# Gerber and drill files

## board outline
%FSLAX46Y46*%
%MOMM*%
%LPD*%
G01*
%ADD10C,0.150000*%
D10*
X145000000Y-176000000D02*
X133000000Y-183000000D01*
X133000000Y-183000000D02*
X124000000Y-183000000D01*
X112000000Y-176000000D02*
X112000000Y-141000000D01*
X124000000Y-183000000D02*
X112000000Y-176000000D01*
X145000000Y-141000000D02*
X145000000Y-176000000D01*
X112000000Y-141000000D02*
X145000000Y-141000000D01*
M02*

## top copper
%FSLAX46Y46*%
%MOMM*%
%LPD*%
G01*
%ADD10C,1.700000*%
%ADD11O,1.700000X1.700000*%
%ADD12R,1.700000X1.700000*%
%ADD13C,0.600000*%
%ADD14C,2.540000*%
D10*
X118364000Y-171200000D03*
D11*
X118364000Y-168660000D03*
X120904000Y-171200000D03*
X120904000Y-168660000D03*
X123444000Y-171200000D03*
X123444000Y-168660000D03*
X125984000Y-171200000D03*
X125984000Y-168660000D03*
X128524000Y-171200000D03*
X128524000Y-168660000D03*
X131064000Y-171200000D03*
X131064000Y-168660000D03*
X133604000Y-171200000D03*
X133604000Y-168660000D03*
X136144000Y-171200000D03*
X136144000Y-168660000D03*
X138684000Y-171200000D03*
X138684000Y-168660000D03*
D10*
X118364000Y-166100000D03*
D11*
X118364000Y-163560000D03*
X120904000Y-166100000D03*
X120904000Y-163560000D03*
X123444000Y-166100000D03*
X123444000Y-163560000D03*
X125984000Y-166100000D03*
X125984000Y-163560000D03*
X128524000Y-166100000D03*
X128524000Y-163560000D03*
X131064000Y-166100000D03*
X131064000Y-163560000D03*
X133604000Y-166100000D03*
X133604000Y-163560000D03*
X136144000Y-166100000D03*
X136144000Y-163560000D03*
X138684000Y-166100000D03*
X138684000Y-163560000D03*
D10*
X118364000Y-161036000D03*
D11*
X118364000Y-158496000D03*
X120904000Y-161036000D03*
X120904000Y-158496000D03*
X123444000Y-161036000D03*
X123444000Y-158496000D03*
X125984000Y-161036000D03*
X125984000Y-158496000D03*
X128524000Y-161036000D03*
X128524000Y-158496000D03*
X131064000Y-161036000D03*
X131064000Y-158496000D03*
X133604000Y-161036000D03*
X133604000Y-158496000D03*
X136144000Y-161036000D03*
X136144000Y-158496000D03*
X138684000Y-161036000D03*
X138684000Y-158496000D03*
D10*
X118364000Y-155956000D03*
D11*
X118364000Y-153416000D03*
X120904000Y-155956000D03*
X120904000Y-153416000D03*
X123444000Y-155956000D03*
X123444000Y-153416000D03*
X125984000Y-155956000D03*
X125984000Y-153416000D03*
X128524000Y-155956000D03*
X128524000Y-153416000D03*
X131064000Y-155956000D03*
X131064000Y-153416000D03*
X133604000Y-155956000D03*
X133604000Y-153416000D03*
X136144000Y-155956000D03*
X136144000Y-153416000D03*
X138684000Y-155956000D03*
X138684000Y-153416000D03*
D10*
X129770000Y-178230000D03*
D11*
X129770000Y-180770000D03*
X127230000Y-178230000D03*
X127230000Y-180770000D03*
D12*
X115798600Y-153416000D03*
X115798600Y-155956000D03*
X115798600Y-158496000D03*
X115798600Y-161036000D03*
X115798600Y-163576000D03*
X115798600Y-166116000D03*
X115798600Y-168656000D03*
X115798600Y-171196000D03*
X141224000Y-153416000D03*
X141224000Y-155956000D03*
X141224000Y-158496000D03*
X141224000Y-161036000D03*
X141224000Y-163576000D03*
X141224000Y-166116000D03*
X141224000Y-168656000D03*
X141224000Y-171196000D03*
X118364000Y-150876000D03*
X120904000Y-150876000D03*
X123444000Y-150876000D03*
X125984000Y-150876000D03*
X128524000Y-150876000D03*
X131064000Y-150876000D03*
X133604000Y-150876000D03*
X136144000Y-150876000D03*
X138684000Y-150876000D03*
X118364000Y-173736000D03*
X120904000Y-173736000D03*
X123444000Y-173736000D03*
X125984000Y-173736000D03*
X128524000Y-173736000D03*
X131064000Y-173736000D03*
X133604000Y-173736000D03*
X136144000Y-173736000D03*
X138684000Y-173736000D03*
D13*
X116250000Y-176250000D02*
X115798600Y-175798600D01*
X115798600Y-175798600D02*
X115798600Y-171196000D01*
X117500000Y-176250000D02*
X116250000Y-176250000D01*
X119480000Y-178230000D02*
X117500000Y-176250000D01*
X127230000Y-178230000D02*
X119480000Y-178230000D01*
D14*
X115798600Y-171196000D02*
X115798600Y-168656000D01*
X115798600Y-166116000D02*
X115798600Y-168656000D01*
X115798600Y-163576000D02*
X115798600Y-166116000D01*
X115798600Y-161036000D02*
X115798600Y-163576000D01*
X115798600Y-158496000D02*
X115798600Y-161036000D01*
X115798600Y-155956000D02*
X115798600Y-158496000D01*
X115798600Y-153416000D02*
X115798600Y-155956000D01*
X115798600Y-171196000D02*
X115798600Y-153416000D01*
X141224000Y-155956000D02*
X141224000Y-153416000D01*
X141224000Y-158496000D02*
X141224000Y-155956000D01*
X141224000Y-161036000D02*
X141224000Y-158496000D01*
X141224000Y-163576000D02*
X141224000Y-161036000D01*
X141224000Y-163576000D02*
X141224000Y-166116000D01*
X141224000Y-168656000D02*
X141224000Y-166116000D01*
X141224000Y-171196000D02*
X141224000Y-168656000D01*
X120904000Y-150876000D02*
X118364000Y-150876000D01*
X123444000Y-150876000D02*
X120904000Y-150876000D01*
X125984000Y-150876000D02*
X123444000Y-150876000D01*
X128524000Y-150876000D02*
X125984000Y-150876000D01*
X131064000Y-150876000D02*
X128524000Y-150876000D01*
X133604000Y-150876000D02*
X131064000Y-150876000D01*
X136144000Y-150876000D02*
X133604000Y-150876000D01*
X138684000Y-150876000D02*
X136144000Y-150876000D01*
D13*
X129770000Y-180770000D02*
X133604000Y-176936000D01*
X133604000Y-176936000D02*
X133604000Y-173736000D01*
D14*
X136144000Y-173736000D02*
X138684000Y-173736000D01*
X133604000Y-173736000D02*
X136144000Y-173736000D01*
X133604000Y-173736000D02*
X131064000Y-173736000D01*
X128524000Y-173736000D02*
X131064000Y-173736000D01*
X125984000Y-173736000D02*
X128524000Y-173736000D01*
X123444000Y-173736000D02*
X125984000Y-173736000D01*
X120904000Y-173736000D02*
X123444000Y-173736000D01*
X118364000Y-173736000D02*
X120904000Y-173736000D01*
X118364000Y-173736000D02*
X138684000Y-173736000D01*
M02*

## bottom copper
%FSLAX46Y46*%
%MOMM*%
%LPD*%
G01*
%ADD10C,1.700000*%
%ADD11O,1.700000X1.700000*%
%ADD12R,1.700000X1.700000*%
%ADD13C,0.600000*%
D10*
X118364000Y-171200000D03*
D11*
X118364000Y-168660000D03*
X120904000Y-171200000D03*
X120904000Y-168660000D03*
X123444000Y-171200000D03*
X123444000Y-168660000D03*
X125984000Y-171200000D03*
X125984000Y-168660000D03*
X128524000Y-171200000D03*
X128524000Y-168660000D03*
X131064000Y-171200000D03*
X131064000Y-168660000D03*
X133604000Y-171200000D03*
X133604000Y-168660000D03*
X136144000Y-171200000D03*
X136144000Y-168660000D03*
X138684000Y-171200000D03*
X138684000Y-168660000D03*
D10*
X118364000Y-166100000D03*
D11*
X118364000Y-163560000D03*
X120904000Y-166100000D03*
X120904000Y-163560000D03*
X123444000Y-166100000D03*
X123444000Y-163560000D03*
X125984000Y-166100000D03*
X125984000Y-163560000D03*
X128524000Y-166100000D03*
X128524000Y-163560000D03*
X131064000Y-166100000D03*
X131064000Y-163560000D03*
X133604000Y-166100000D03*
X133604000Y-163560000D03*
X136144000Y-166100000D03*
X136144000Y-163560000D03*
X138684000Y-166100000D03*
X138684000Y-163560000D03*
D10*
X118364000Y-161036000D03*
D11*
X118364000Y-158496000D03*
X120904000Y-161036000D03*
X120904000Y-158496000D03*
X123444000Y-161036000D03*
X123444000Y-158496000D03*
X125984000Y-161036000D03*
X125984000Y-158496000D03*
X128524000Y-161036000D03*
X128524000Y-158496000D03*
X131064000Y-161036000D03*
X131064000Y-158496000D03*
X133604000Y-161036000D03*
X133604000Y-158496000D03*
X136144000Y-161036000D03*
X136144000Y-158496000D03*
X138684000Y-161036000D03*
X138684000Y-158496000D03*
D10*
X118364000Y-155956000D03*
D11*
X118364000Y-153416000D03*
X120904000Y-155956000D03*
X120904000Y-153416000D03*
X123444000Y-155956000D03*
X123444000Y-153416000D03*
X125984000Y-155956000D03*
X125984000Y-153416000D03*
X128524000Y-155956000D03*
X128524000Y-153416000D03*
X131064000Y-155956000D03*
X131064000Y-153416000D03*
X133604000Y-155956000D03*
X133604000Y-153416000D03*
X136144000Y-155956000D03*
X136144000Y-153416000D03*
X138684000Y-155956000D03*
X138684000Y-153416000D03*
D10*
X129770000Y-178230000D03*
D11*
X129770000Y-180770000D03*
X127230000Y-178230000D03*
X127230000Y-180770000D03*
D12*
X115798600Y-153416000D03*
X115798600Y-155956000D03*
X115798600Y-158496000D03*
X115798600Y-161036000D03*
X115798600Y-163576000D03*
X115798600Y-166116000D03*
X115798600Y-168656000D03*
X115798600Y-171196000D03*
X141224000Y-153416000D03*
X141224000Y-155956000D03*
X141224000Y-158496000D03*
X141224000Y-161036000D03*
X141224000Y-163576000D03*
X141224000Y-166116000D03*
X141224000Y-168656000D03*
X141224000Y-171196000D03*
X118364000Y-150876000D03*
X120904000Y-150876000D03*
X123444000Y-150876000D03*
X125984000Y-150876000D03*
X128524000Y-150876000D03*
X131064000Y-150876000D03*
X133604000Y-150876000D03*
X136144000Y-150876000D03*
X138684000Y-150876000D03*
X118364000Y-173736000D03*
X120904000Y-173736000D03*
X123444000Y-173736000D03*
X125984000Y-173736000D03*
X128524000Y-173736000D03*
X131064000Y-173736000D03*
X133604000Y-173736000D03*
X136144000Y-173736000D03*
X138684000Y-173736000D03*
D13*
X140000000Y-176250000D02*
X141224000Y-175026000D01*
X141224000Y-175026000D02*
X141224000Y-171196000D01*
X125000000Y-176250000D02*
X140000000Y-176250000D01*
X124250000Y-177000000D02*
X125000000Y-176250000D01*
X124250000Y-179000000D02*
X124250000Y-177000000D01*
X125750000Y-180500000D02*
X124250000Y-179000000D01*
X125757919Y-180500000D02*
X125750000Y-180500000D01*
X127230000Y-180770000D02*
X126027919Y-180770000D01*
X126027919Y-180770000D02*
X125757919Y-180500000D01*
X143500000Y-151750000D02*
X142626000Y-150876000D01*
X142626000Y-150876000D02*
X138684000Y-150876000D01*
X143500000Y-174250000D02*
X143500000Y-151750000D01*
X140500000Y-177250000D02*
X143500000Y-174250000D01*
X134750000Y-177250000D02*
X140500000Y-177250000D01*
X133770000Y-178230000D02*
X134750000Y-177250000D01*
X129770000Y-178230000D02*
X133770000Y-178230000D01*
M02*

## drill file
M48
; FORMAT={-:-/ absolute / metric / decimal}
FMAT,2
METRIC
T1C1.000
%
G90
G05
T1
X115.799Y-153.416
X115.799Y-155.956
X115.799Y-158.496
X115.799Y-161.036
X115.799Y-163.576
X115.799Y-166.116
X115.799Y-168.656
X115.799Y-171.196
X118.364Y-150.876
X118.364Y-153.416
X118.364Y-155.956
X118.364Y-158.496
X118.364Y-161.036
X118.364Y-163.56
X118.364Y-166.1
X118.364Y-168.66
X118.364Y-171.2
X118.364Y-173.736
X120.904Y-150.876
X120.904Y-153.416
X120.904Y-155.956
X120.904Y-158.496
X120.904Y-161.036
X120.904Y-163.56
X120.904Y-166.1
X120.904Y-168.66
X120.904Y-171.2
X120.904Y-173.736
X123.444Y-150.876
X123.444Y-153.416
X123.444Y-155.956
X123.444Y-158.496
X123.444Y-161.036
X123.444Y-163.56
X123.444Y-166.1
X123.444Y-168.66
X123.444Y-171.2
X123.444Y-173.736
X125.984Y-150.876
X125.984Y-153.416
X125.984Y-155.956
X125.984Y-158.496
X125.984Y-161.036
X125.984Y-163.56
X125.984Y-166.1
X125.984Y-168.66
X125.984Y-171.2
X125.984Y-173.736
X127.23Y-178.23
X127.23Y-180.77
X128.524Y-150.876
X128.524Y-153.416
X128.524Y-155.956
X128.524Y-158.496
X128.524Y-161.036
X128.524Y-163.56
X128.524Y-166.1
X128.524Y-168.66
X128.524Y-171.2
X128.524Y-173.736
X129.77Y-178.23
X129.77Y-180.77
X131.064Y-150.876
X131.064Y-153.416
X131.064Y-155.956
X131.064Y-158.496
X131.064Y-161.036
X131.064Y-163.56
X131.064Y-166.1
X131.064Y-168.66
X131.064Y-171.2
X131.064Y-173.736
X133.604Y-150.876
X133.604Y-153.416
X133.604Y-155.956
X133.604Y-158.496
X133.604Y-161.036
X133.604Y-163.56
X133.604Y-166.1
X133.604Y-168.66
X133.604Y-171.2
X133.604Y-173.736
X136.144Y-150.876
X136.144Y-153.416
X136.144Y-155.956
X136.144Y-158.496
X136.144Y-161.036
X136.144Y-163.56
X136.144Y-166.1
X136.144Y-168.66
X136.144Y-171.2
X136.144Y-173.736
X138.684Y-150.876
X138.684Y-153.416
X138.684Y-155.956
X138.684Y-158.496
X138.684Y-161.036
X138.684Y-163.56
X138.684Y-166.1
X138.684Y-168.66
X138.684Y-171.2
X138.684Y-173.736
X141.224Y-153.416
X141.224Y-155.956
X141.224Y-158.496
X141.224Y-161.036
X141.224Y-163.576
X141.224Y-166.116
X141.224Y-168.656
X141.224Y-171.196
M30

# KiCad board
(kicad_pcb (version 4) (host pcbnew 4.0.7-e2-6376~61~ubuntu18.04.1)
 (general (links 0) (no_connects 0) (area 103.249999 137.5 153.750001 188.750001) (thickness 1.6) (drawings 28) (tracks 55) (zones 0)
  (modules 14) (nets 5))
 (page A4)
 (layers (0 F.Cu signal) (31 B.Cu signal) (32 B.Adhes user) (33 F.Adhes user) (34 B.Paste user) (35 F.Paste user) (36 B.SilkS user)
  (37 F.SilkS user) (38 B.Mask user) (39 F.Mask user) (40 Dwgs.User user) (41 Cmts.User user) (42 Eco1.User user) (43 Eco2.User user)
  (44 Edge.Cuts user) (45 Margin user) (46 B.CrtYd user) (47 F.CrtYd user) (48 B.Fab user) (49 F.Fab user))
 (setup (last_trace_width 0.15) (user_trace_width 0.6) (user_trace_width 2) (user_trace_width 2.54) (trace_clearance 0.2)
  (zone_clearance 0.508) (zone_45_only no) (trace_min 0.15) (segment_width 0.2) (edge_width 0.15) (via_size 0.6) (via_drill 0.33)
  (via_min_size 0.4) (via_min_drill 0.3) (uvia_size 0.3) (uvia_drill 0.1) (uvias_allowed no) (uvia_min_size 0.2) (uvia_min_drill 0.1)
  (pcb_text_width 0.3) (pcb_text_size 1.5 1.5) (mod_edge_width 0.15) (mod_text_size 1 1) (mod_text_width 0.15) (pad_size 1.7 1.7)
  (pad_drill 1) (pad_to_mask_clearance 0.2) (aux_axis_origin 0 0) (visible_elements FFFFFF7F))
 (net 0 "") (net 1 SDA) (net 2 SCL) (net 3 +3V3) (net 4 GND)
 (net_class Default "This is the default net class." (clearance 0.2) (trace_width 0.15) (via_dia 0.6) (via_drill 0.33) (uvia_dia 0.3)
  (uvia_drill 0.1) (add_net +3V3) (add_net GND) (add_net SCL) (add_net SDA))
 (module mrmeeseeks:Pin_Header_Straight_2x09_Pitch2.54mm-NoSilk (layer F.Cu) (at 118.364 171.2 90)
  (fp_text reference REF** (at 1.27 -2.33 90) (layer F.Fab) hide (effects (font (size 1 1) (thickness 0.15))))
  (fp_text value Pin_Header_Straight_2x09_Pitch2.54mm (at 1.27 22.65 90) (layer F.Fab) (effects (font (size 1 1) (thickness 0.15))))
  (pad 1 thru_hole circle (at 0 0 90) (size 1.7 1.7) (drill 1) (layers *.Cu *.Mask))
  (pad 2 thru_hole oval (at 2.54 0 90) (size 1.7 1.7) (drill 1) (layers *.Cu *.Mask))
  (pad 3 thru_hole oval (at 0 2.54 90) (size 1.7 1.7) (drill 1) (layers *.Cu *.Mask))
  (pad 4 thru_hole oval (at 2.54 2.54 90) (size 1.7 1.7) (drill 1) (layers *.Cu *.Mask))
  (pad 5 thru_hole oval (at 0 5.08 90) (size 1.7 1.7) (drill 1) (layers *.Cu *.Mask))
  (pad 6 thru_hole oval (at 2.54 5.08 90) (size 1.7 1.7) (drill 1) (layers *.Cu *.Mask))
  (pad 7 thru_hole oval (at 0 7.62 90) (size 1.7 1.7) (drill 1) (layers *.Cu *.Mask))
  (pad 8 thru_hole oval (at 2.54 7.62 90) (size 1.7 1.7) (drill 1) (layers *.Cu *.Mask))
  (pad 9 thru_hole oval (at 0 10.16 90) (size 1.7 1.7) (drill 1) (layers *.Cu *.Mask))
  (pad 10 thru_hole oval (at 2.54 10.16 90) (size 1.7 1.7) (drill 1) (layers *.Cu *.Mask))
  (pad 11 thru_hole oval (at 0 12.7 90) (size 1.7 1.7) (drill 1) (layers *.Cu *.Mask))
  (pad 12 thru_hole oval (at 2.54 12.7 90) (size 1.7 1.7) (drill 1) (layers *.Cu *.Mask))
  (pad 13 thru_hole oval (at 0 15.24 90) (size 1.7 1.7) (drill 1) (layers *.Cu *.Mask))
  (pad 14 thru_hole oval (at 2.54 15.24 90) (size 1.7 1.7) (drill 1) (layers *.Cu *.Mask))
  (pad 15 thru_hole oval (at 0 17.78 90) (size 1.7 1.7) (drill 1) (layers *.Cu *.Mask))
  (pad 16 thru_hole oval (at 2.54 17.78 90) (size 1.7 1.7) (drill 1) (layers *.Cu *.Mask))
  (pad 17 thru_hole oval (at 0 20.32 90) (size 1.7 1.7) (drill 1) (layers *.Cu *.Mask))
  (pad 18 thru_hole oval (at 2.54 20.32 90) (size 1.7 1.7) (drill 1) (layers *.Cu *.Mask)))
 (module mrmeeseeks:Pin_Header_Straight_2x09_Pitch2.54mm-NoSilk (layer F.Cu) (at 118.364 166.1 90)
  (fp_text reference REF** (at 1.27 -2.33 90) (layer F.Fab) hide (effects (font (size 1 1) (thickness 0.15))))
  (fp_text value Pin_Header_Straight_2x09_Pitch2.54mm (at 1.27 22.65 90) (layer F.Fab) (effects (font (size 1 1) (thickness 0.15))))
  (pad 1 thru_hole circle (at 0 0 90) (size 1.7 1.7) (drill 1) (layers *.Cu *.Mask))
  (pad 2 thru_hole oval (at 2.54 0 90) (size 1.7 1.7) (drill 1) (layers *.Cu *.Mask))
  (pad 3 thru_hole oval (at 0 2.54 90) (size 1.7 1.7) (drill 1) (layers *.Cu *.Mask))
  (pad 4 thru_hole oval (at 2.54 2.54 90) (size 1.7 1.7) (drill 1) (layers *.Cu *.Mask))
  (pad 5 thru_hole oval (at 0 5.08 90) (size 1.7 1.7) (drill 1) (layers *.Cu *.Mask))
  (pad 6 thru_hole oval (at 2.54 5.08 90) (size 1.7 1.7) (drill 1) (layers *.Cu *.Mask))
  (pad 7 thru_hole oval (at 0 7.62 90) (size 1.7 1.7) (drill 1) (layers *.Cu *.Mask))
  (pad 8 thru_hole oval (at 2.54 7.62 90) (size 1.7 1.7) (drill 1) (layers *.Cu *.Mask))
  (pad 9 thru_hole oval (at 0 10.16 90) (size 1.7 1.7) (drill 1) (layers *.Cu *.Mask))
  (pad 10 thru_hole oval (at 2.54 10.16 90) (size 1.7 1.7) (drill 1) (layers *.Cu *.Mask))
  (pad 11 thru_hole oval (at 0 12.7 90) (size 1.7 1.7) (drill 1) (layers *.Cu *.Mask))
  (pad 12 thru_hole oval (at 2.54 12.7 90) (size 1.7 1.7) (drill 1) (layers *.Cu *.Mask))
  (pad 13 thru_hole oval (at 0 15.24 90) (size 1.7 1.7) (drill 1) (layers *.Cu *.Mask))
  (pad 14 thru_hole oval (at 2.54 15.24 90) (size 1.7 1.7) (drill 1) (layers *.Cu *.Mask))
  (pad 15 thru_hole oval (at 0 17.78 90) (size 1.7 1.7) (drill 1) (layers *.Cu *.Mask))
  (pad 16 thru_hole oval (at 2.54 17.78 90) (size 1.7 1.7) (drill 1) (layers *.Cu *.Mask))
  (pad 17 thru_hole oval (at 0 20.32 90) (size 1.7 1.7) (drill 1) (layers *.Cu *.Mask))
  (pad 18 thru_hole oval (at 2.54 20.32 90) (size 1.7 1.7) (drill 1) (layers *.Cu *.Mask)))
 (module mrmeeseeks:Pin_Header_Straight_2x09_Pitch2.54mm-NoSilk (layer F.Cu) (at 118.364 161.036 90)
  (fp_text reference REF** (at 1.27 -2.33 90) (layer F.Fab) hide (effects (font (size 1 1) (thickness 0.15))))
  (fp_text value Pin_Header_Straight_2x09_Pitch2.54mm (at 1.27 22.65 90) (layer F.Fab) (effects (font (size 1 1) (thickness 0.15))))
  (pad 1 thru_hole circle (at 0 0 90) (size 1.7 1.7) (drill 1) (layers *.Cu *.Mask))
  (pad 2 thru_hole oval (at 2.54 0 90) (size 1.7 1.7) (drill 1) (layers *.Cu *.Mask))
  (pad 3 thru_hole oval (at 0 2.54 90) (size 1.7 1.7) (drill 1) (layers *.Cu *.Mask))
  (pad 4 thru_hole oval (at 2.54 2.54 90) (size 1.7 1.7) (drill 1) (layers *.Cu *.Mask))
  (pad 5 thru_hole oval (at 0 5.08 90) (size 1.7 1.7) (drill 1) (layers *.Cu *.Mask))
  (pad 6 thru_hole oval (at 2.54 5.08 90) (size 1.7 1.7) (drill 1) (layers *.Cu *.Mask))
  (pad 7 thru_hole oval (at 0 7.62 90) (size 1.7 1.7) (drill 1) (layers *.Cu *.Mask))
  (pad 8 thru_hole oval (at 2.54 7.62 90) (size 1.7 1.7) (drill 1) (layers *.Cu *.Mask))
  (pad 9 thru_hole oval (at 0 10.16 90) (size 1.7 1.7) (drill 1) (layers *.Cu *.Mask))
  (pad 10 thru_hole oval (at 2.54 10.16 90) (size 1.7 1.7) (drill 1) (layers *.Cu *.Mask))
  (pad 11 thru_hole oval (at 0 12.7 90) (size 1.7 1.7) (drill 1) (layers *.Cu *.Mask))
  (pad 12 thru_hole oval (at 2.54 12.7 90) (size 1.7 1.7) (drill 1) (layers *.Cu *.Mask))
  (pad 13 thru_hole oval (at 0 15.24 90) (size 1.7 1.7) (drill 1) (layers *.Cu *.Mask))
  (pad 14 thru_hole oval (at 2.54 15.24 90) (size 1.7 1.7) (drill 1) (layers *.Cu *.Mask))
  (pad 15 thru_hole oval (at 0 17.78 90) (size 1.7 1.7) (drill 1) (layers *.Cu *.Mask))
  (pad 16 thru_hole oval (at 2.54 17.78 90) (size 1.7 1.7) (drill 1) (layers *.Cu *.Mask))
  (pad 17 thru_hole oval (at 0 20.32 90) (size 1.7 1.7) (drill 1) (layers *.Cu *.Mask))
  (pad 18 thru_hole oval (at 2.54 20.32 90) (size 1.7 1.7) (drill 1) (layers *.Cu *.Mask)))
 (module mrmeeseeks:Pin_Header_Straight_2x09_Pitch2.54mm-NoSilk (layer F.Cu) (at 118.364 155.956 90)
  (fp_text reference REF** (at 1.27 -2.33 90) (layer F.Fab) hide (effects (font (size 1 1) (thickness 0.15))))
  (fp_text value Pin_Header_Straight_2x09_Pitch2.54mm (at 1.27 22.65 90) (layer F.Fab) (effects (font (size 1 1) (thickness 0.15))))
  (pad 1 thru_hole circle (at 0 0 90) (size 1.7 1.7) (drill 1) (layers *.Cu *.Mask))
  (pad 2 thru_hole oval (at 2.54 0 90) (size 1.7 1.7) (drill 1) (layers *.Cu *.Mask))
  (pad 3 thru_hole oval (at 0 2.54 90) (size 1.7 1.7) (drill 1) (layers *.Cu *.Mask))
  (pad 4 thru_hole oval (at 2.54 2.54 90) (size 1.7 1.7) (drill 1) (layers *.Cu *.Mask))
  (pad 5 thru_hole oval (at 0 5.08 90) (size 1.7 1.7) (drill 1) (layers *.Cu *.Mask))
  (pad 6 thru_hole oval (at 2.54 5.08 90) (size 1.7 1.7) (drill 1) (layers *.Cu *.Mask))
  (pad 7 thru_hole oval (at 0 7.62 90) (size 1.7 1.7) (drill 1) (layers *.Cu *.Mask))
  (pad 8 thru_hole oval (at 2.54 7.62 90) (size 1.7 1.7) (drill 1) (layers *.Cu *.Mask))
  (pad 9 thru_hole oval (at 0 10.16 90) (size 1.7 1.7) (drill 1) (layers *.Cu *.Mask))
  (pad 10 thru_hole oval (at 2.54 10.16 90) (size 1.7 1.7) (drill 1) (layers *.Cu *.Mask))
  (pad 11 thru_hole oval (at 0 12.7 90) (size 1.7 1.7) (drill 1) (layers *.Cu *.Mask))
  (pad 12 thru_hole oval (at 2.54 12.7 90) (size 1.7 1.7) (drill 1) (layers *.Cu *.Mask))
  (pad 13 thru_hole oval (at 0 15.24 90) (size 1.7 1.7) (drill 1) (layers *.Cu *.Mask))
  (pad 14 thru_hole oval (at 2.54 15.24 90) (size 1.7 1.7) (drill 1) (layers *.Cu *.Mask))
  (pad 15 thru_hole oval (at 0 17.78 90) (size 1.7 1.7) (drill 1) (layers *.Cu *.Mask))
  (pad 16 thru_hole oval (at 2.54 17.78 90) (size 1.7 1.7) (drill 1) (layers *.Cu *.Mask))
  (pad 17 thru_hole oval (at 0 20.32 90) (size 1.7 1.7) (drill 1) (layers *.Cu *.Mask))
  (pad 18 thru_hole oval (at 2.54 20.32 90) (size 1.7 1.7) (drill 1) (layers *.Cu *.Mask)))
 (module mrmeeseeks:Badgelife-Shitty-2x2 (layer F.Cu) (at 128.5 179.5)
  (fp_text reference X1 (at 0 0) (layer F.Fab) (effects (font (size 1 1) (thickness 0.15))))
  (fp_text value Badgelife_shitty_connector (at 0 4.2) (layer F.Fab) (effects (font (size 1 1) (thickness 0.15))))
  (pad 4 thru_hole circle (at 1.27 -1.27) (size 1.7 1.7) (drill 1) (layers *.Cu *.Mask) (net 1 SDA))
  (pad 3 thru_hole oval (at 1.27 1.27) (size 1.7 1.7) (drill 1) (layers *.Cu *.Mask) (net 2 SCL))
  (pad 1 thru_hole oval (at -1.27 -1.27) (size 1.7 1.7) (drill 1) (layers *.Cu *.Mask) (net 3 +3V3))
  (pad 2 thru_hole oval (at -1.27 1.27) (size 1.7 1.7) (drill 1) (layers *.Cu *.Mask) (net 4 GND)))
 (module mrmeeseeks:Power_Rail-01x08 (layer F.Cu) (at 115.7986 153.416)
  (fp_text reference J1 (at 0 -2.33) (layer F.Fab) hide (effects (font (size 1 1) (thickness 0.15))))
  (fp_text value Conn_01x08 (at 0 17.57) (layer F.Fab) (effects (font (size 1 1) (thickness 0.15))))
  (pad 1 thru_hole rect (at 0 0) (size 1.7 1.7) (drill 1) (layers *.Cu *.Mask) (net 3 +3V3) (solder_mask_margin 0.1))
  (pad 2 thru_hole rect (at 0 2.54) (size 1.7 1.7) (drill 1) (layers *.Cu *.Mask) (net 3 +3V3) (solder_mask_margin 0.1))
  (pad 3 thru_hole rect (at 0 5.08) (size 1.7 1.7) (drill 1) (layers *.Cu *.Mask) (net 3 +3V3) (solder_mask_margin 0.1))
  (pad 4 thru_hole rect (at 0 7.62) (size 1.7 1.7) (drill 1) (layers *.Cu *.Mask) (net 3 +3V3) (solder_mask_margin 0.1))
  (pad 5 thru_hole rect (at 0 10.16) (size 1.7 1.7) (drill 1) (layers *.Cu *.Mask) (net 3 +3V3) (solder_mask_margin 0.1))
  (pad 6 thru_hole rect (at 0 12.7) (size 1.7 1.7) (drill 1) (layers *.Cu *.Mask) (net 3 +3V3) (solder_mask_margin 0.1))
  (pad 7 thru_hole rect (at 0 15.24) (size 1.7 1.7) (drill 1) (layers *.Cu *.Mask) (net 3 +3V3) (solder_mask_margin 0.1))
  (pad 8 thru_hole rect (at 0 17.78) (size 1.7 1.7) (drill 1) (layers *.Cu *.Mask) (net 3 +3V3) (solder_mask_margin 0.1)))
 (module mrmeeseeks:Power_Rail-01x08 (layer F.Cu) (at 141.224 153.416)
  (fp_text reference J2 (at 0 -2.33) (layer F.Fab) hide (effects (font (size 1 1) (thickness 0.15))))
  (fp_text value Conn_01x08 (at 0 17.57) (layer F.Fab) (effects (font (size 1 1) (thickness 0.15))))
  (pad 1 thru_hole rect (at 0 0) (size 1.7 1.7) (drill 1) (layers *.Cu *.Mask) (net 4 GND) (solder_mask_margin 0.1))
  (pad 2 thru_hole rect (at 0 2.54) (size 1.7 1.7) (drill 1) (layers *.Cu *.Mask) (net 4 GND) (solder_mask_margin 0.1))
  (pad 3 thru_hole rect (at 0 5.08) (size 1.7 1.7) (drill 1) (layers *.Cu *.Mask) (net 4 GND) (solder_mask_margin 0.1))
  (pad 4 thru_hole rect (at 0 7.62) (size 1.7 1.7) (drill 1) (layers *.Cu *.Mask) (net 4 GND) (solder_mask_margin 0.1))
  (pad 5 thru_hole rect (at 0 10.16) (size 1.7 1.7) (drill 1) (layers *.Cu *.Mask) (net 4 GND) (solder_mask_margin 0.1))
  (pad 6 thru_hole rect (at 0 12.7) (size 1.7 1.7) (drill 1) (layers *.Cu *.Mask) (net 4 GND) (solder_mask_margin 0.1))
  (pad 7 thru_hole rect (at 0 15.24) (size 1.7 1.7) (drill 1) (layers *.Cu *.Mask) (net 4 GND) (solder_mask_margin 0.1))
  (pad 8 thru_hole rect (at 0 17.78) (size 1.7 1.7) (drill 1) (layers *.Cu *.Mask) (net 4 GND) (solder_mask_margin 0.1)))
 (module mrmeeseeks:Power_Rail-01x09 (layer F.Cu) (at 118.364 150.876 90)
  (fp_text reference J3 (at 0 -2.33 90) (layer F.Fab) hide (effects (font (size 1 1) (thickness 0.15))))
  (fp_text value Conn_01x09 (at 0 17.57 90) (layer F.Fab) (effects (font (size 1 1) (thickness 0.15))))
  (pad 1 thru_hole rect (at 0 0 90) (size 1.7 1.7) (drill 1) (layers *.Cu *.Mask) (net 1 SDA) (solder_mask_margin 0.1))
  (pad 2 thru_hole rect (at 0 2.54 90) (size 1.7 1.7) (drill 1) (layers *.Cu *.Mask) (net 1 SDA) (solder_mask_margin 0.1))
  (pad 3 thru_hole rect (at 0 5.08 90) (size 1.7 1.7) (drill 1) (layers *.Cu *.Mask) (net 1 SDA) (solder_mask_margin 0.1))
  (pad 4 thru_hole rect (at 0 7.62 90) (size 1.7 1.7) (drill 1) (layers *.Cu *.Mask) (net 1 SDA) (solder_mask_margin 0.1))
  (pad 5 thru_hole rect (at 0 10.16 90) (size 1.7 1.7) (drill 1) (layers *.Cu *.Mask) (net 1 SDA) (solder_mask_margin 0.1))
  (pad 6 thru_hole rect (at 0 12.7 90) (size 1.7 1.7) (drill 1) (layers *.Cu *.Mask) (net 1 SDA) (solder_mask_margin 0.1))
  (pad 7 thru_hole rect (at 0 15.24 90) (size 1.7 1.7) (drill 1) (layers *.Cu *.Mask) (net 1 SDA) (solder_mask_margin 0.1))
  (pad 8 thru_hole rect (at 0 17.78 90) (size 1.7 1.7) (drill 1) (layers *.Cu *.Mask) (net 1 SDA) (solder_mask_margin 0.1))
  (pad 9 thru_hole rect (at 0 20.32 90) (size 1.7 1.7) (drill 1) (layers *.Cu *.Mask) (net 1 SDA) (solder_mask_margin 0.1)))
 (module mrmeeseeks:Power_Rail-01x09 (layer F.Cu) (at 118.364 173.736 90)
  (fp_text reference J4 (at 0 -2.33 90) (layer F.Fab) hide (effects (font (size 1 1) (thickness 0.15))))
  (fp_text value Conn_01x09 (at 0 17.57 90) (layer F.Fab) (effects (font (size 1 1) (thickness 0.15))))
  (pad 1 thru_hole rect (at 0 0 90) (size 1.7 1.7) (drill 1) (layers *.Cu *.Mask) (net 2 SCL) (solder_mask_margin 0.1))
  (pad 2 thru_hole rect (at 0 2.54 90) (size 1.7 1.7) (drill 1) (layers *.Cu *.Mask) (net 2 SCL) (solder_mask_margin 0.1))
  (pad 3 thru_hole rect (at 0 5.08 90) (size 1.7 1.7) (drill 1) (layers *.Cu *.Mask) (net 2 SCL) (solder_mask_margin 0.1))
  (pad 4 thru_hole rect (at 0 7.62 90) (size 1.7 1.7) (drill 1) (layers *.Cu *.Mask) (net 2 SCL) (solder_mask_margin 0.1))
  (pad 5 thru_hole rect (at 0 10.16 90) (size 1.7 1.7) (drill 1) (layers *.Cu *.Mask) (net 2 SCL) (solder_mask_margin 0.1))
  (pad 6 thru_hole rect (at 0 12.7 90) (size 1.7 1.7) (drill 1) (layers *.Cu *.Mask) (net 2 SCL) (solder_mask_margin 0.1))
  (pad 7 thru_hole rect (at 0 15.24 90) (size 1.7 1.7) (drill 1) (layers *.Cu *.Mask) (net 2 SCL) (solder_mask_margin 0.1))
  (pad 8 thru_hole rect (at 0 17.78 90) (size 1.7 1.7) (drill 1) (layers *.Cu *.Mask) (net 2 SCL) (solder_mask_margin 0.1))
  (pad 9 thru_hole rect (at 0 20.32 90) (size 1.7 1.7) (drill 1) (layers *.Cu *.Mask) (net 2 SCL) (solder_mask_margin 0.1)))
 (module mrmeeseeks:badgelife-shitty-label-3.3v (layer F.Cu) (at 113.4 162.2 90)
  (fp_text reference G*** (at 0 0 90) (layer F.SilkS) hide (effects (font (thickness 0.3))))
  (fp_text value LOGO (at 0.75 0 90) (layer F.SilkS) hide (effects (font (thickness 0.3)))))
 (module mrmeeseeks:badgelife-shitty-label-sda (layer F.Cu) (at 128.2 148.8)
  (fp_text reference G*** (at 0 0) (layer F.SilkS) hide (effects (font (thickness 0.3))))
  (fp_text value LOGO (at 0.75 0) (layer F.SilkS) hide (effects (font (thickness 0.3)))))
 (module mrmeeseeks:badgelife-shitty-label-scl (layer F.Cu) (at 128.4 175.7)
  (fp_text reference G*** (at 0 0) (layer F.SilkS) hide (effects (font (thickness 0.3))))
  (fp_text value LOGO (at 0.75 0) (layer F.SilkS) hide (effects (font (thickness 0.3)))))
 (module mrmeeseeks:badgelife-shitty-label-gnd (layer F.Cu) (at 143.7 162.3 270)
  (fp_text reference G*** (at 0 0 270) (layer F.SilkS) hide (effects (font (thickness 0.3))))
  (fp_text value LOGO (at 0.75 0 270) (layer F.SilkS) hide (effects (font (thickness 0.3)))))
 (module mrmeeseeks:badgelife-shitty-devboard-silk (layer F.Cu) (at 128.9 144.6)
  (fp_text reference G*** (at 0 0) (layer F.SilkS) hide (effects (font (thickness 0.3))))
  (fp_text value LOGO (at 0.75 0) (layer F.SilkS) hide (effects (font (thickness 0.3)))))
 (gr_line (start 145 176) (end 133 183) (layer Edge.Cuts) (width 0.15))
 (gr_line (start 133 183) (end 124 183) (layer Edge.Cuts) (width 0.15))
 (gr_line (start 112 176) (end 112 141) (layer Edge.Cuts) (width 0.15))
 (gr_line (start 124 183) (end 112 176) (layer Edge.Cuts) (width 0.15))
 (gr_line (start 145 141) (end 145 176) (layer Edge.Cuts) (width 0.15))
 (gr_line (start 112 141) (end 145 141) (layer Edge.Cuts) (width 0.15))
 (segment (start 116.25 176.25) (end 115.7986 175.7986) (width 0.6) (layer F.Cu) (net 3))
 (segment (start 115.7986 175.7986) (end 115.7986 171.196) (width 0.6) (layer F.Cu) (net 3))
 (segment (start 117.5 176.25) (end 116.25 176.25) (width 0.6) (layer F.Cu) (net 3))
 (segment (start 119.48 178.23) (end 117.5 176.25) (width 0.6) (layer F.Cu) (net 3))
 (segment (start 127.23 178.23) (end 119.48 178.23) (width 0.6) (layer F.Cu) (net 3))
 (segment (start 115.7986 171.196) (end 115.7986 168.656) (width 2.54) (layer F.Cu) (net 3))
 (segment (start 115.7986 166.116) (end 115.7986 168.656) (width 2.54) (layer F.Cu) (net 3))
 (segment (start 115.7986 163.576) (end 115.7986 166.116) (width 2.54) (layer F.Cu) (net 3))
 (segment (start 115.7986 161.036) (end 115.7986 163.576) (width 2.54) (layer F.Cu) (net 3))
 (segment (start 115.7986 158.496) (end 115.7986 161.036) (width 2.54) (layer F.Cu) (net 3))
 (segment (start 115.7986 155.956) (end 115.7986 158.496) (width 2.54) (layer F.Cu) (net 3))
 (segment (start 115.7986 153.416) (end 115.7986 155.956) (width 2.54) (layer F.Cu) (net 3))
 (segment (start 115.7986 171.196) (end 115.7986 153.416) (width 2.54) (layer F.Cu) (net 3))
 (segment (start 140 176.25) (end 141.224 175.026) (width 0.6) (layer B.Cu) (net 4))
 (segment (start 141.224 175.026) (end 141.224 171.196) (width 0.6) (layer B.Cu) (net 4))
 (segment (start 125 176.25) (end 140 176.25) (width 0.6) (layer B.Cu) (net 4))
 (segment (start 124.25 177) (end 125 176.25) (width 0.6) (layer B.Cu) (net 4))
 (segment (start 124.25 179) (end 124.25 177) (width 0.6) (layer B.Cu) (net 4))
 (segment (start 125.75 180.5) (end 124.25 179) (width 0.6) (layer B.Cu) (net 4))
 (segment (start 125.757919 180.5) (end 125.75 180.5) (width 0.6) (layer B.Cu) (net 4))
 (segment (start 127.23 180.77) (end 126.027919 180.77) (width 0.6) (layer B.Cu) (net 4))
 (segment (start 126.027919 180.77) (end 125.757919 180.5) (width 0.6) (layer B.Cu) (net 4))
 (segment (start 141.224 155.956) (end 141.224 153.416) (width 2.54) (layer F.Cu) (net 4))
 (segment (start 141.224 158.496) (end 141.224 155.956) (width 2.54) (layer F.Cu) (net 4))
 (segment (start 141.224 161.036) (end 141.224 158.496) (width 2.54) (layer F.Cu) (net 4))
 (segment (start 141.224 163.576) (end 141.224 161.036) (width 2.54) (layer F.Cu) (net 4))
 (segment (start 141.224 163.576) (end 141.224 166.116) (width 2.54) (layer F.Cu) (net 4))
 (segment (start 141.224 168.656) (end 141.224 166.116) (width 2.54) (layer F.Cu) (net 4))
 (segment (start 141.224 171.196) (end 141.224 168.656) (width 2.54) (layer F.Cu) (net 4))
 (segment (start 143.5 151.75) (end 142.626 150.876) (width 0.6) (layer B.Cu) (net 1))
 (segment (start 142.626 150.876) (end 138.684 150.876) (width 0.6) (layer B.Cu) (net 1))
 (segment (start 143.5 174.25) (end 143.5 151.75) (width 0.6) (layer B.Cu) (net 1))
 (segment (start 140.5 177.25) (end 143.5 174.25) (width 0.6) (layer B.Cu) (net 1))
 (segment (start 134.75 177.25) (end 140.5 177.25) (width 0.6) (layer B.Cu) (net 1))
 (segment (start 133.77 178.23) (end 134.75 177.25) (width 0.6) (layer B.Cu) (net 1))
 (segment (start 129.77 178.23) (end 133.77 178.23) (width 0.6) (layer B.Cu) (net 1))
 (segment (start 120.904 150.876) (end 118.364 150.876) (width 2.54) (layer F.Cu) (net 1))
 (segment (start 123.444 150.876) (end 120.904 150.876) (width 2.54) (layer F.Cu) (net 1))
 (segment (start 125.984 150.876) (end 123.444 150.876) (width 2.54) (layer F.Cu) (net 1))
 (segment (start 128.524 150.876) (end 125.984 150.876) (width 2.54) (layer F.Cu) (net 1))
 (segment (start 131.064 150.876) (end 128.524 150.876) (width 2.54) (layer F.Cu) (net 1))
 (segment (start 133.604 150.876) (end 131.064 150.876) (width 2.54) (layer F.Cu) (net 1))
 (segment (start 136.144 150.876) (end 133.604 150.876) (width 2.54) (layer F.Cu) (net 1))
 (segment (start 138.684 150.876) (end 136.144 150.876) (width 2.54) (layer F.Cu) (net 1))
 (segment (start 129.77 180.77) (end 133.604 176.936) (width 0.6) (layer F.Cu) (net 2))
 (segment (start 133.604 176.936) (end 133.604 173.736) (width 0.6) (layer F.Cu) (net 2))
 (segment (start 136.144 173.736) (end 138.684 173.736) (width 2.54) (layer F.Cu) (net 2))
 (segment (start 133.604 173.736) (end 136.144 173.736) (width 2.54) (layer F.Cu) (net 2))
 (segment (start 133.604 173.736) (end 131.064 173.736) (width 2.54) (layer F.Cu) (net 2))
 (segment (start 128.524 173.736) (end 131.064 173.736) (width 2.54) (layer F.Cu) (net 2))
 (segment (start 125.984 173.736) (end 128.524 173.736) (width 2.54) (layer F.Cu) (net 2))
 (segment (start 123.444 173.736) (end 125.984 173.736) (width 2.54) (layer F.Cu) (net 2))
 (segment (start 120.904 173.736) (end 123.444 173.736) (width 2.54) (layer F.Cu) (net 2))
 (segment (start 118.364 173.736) (end 120.904 173.736) (width 2.54) (layer F.Cu) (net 2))
 (segment (start 118.364 173.736) (end 138.684 173.736) (width 2.54) (layer F.Cu) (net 2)))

